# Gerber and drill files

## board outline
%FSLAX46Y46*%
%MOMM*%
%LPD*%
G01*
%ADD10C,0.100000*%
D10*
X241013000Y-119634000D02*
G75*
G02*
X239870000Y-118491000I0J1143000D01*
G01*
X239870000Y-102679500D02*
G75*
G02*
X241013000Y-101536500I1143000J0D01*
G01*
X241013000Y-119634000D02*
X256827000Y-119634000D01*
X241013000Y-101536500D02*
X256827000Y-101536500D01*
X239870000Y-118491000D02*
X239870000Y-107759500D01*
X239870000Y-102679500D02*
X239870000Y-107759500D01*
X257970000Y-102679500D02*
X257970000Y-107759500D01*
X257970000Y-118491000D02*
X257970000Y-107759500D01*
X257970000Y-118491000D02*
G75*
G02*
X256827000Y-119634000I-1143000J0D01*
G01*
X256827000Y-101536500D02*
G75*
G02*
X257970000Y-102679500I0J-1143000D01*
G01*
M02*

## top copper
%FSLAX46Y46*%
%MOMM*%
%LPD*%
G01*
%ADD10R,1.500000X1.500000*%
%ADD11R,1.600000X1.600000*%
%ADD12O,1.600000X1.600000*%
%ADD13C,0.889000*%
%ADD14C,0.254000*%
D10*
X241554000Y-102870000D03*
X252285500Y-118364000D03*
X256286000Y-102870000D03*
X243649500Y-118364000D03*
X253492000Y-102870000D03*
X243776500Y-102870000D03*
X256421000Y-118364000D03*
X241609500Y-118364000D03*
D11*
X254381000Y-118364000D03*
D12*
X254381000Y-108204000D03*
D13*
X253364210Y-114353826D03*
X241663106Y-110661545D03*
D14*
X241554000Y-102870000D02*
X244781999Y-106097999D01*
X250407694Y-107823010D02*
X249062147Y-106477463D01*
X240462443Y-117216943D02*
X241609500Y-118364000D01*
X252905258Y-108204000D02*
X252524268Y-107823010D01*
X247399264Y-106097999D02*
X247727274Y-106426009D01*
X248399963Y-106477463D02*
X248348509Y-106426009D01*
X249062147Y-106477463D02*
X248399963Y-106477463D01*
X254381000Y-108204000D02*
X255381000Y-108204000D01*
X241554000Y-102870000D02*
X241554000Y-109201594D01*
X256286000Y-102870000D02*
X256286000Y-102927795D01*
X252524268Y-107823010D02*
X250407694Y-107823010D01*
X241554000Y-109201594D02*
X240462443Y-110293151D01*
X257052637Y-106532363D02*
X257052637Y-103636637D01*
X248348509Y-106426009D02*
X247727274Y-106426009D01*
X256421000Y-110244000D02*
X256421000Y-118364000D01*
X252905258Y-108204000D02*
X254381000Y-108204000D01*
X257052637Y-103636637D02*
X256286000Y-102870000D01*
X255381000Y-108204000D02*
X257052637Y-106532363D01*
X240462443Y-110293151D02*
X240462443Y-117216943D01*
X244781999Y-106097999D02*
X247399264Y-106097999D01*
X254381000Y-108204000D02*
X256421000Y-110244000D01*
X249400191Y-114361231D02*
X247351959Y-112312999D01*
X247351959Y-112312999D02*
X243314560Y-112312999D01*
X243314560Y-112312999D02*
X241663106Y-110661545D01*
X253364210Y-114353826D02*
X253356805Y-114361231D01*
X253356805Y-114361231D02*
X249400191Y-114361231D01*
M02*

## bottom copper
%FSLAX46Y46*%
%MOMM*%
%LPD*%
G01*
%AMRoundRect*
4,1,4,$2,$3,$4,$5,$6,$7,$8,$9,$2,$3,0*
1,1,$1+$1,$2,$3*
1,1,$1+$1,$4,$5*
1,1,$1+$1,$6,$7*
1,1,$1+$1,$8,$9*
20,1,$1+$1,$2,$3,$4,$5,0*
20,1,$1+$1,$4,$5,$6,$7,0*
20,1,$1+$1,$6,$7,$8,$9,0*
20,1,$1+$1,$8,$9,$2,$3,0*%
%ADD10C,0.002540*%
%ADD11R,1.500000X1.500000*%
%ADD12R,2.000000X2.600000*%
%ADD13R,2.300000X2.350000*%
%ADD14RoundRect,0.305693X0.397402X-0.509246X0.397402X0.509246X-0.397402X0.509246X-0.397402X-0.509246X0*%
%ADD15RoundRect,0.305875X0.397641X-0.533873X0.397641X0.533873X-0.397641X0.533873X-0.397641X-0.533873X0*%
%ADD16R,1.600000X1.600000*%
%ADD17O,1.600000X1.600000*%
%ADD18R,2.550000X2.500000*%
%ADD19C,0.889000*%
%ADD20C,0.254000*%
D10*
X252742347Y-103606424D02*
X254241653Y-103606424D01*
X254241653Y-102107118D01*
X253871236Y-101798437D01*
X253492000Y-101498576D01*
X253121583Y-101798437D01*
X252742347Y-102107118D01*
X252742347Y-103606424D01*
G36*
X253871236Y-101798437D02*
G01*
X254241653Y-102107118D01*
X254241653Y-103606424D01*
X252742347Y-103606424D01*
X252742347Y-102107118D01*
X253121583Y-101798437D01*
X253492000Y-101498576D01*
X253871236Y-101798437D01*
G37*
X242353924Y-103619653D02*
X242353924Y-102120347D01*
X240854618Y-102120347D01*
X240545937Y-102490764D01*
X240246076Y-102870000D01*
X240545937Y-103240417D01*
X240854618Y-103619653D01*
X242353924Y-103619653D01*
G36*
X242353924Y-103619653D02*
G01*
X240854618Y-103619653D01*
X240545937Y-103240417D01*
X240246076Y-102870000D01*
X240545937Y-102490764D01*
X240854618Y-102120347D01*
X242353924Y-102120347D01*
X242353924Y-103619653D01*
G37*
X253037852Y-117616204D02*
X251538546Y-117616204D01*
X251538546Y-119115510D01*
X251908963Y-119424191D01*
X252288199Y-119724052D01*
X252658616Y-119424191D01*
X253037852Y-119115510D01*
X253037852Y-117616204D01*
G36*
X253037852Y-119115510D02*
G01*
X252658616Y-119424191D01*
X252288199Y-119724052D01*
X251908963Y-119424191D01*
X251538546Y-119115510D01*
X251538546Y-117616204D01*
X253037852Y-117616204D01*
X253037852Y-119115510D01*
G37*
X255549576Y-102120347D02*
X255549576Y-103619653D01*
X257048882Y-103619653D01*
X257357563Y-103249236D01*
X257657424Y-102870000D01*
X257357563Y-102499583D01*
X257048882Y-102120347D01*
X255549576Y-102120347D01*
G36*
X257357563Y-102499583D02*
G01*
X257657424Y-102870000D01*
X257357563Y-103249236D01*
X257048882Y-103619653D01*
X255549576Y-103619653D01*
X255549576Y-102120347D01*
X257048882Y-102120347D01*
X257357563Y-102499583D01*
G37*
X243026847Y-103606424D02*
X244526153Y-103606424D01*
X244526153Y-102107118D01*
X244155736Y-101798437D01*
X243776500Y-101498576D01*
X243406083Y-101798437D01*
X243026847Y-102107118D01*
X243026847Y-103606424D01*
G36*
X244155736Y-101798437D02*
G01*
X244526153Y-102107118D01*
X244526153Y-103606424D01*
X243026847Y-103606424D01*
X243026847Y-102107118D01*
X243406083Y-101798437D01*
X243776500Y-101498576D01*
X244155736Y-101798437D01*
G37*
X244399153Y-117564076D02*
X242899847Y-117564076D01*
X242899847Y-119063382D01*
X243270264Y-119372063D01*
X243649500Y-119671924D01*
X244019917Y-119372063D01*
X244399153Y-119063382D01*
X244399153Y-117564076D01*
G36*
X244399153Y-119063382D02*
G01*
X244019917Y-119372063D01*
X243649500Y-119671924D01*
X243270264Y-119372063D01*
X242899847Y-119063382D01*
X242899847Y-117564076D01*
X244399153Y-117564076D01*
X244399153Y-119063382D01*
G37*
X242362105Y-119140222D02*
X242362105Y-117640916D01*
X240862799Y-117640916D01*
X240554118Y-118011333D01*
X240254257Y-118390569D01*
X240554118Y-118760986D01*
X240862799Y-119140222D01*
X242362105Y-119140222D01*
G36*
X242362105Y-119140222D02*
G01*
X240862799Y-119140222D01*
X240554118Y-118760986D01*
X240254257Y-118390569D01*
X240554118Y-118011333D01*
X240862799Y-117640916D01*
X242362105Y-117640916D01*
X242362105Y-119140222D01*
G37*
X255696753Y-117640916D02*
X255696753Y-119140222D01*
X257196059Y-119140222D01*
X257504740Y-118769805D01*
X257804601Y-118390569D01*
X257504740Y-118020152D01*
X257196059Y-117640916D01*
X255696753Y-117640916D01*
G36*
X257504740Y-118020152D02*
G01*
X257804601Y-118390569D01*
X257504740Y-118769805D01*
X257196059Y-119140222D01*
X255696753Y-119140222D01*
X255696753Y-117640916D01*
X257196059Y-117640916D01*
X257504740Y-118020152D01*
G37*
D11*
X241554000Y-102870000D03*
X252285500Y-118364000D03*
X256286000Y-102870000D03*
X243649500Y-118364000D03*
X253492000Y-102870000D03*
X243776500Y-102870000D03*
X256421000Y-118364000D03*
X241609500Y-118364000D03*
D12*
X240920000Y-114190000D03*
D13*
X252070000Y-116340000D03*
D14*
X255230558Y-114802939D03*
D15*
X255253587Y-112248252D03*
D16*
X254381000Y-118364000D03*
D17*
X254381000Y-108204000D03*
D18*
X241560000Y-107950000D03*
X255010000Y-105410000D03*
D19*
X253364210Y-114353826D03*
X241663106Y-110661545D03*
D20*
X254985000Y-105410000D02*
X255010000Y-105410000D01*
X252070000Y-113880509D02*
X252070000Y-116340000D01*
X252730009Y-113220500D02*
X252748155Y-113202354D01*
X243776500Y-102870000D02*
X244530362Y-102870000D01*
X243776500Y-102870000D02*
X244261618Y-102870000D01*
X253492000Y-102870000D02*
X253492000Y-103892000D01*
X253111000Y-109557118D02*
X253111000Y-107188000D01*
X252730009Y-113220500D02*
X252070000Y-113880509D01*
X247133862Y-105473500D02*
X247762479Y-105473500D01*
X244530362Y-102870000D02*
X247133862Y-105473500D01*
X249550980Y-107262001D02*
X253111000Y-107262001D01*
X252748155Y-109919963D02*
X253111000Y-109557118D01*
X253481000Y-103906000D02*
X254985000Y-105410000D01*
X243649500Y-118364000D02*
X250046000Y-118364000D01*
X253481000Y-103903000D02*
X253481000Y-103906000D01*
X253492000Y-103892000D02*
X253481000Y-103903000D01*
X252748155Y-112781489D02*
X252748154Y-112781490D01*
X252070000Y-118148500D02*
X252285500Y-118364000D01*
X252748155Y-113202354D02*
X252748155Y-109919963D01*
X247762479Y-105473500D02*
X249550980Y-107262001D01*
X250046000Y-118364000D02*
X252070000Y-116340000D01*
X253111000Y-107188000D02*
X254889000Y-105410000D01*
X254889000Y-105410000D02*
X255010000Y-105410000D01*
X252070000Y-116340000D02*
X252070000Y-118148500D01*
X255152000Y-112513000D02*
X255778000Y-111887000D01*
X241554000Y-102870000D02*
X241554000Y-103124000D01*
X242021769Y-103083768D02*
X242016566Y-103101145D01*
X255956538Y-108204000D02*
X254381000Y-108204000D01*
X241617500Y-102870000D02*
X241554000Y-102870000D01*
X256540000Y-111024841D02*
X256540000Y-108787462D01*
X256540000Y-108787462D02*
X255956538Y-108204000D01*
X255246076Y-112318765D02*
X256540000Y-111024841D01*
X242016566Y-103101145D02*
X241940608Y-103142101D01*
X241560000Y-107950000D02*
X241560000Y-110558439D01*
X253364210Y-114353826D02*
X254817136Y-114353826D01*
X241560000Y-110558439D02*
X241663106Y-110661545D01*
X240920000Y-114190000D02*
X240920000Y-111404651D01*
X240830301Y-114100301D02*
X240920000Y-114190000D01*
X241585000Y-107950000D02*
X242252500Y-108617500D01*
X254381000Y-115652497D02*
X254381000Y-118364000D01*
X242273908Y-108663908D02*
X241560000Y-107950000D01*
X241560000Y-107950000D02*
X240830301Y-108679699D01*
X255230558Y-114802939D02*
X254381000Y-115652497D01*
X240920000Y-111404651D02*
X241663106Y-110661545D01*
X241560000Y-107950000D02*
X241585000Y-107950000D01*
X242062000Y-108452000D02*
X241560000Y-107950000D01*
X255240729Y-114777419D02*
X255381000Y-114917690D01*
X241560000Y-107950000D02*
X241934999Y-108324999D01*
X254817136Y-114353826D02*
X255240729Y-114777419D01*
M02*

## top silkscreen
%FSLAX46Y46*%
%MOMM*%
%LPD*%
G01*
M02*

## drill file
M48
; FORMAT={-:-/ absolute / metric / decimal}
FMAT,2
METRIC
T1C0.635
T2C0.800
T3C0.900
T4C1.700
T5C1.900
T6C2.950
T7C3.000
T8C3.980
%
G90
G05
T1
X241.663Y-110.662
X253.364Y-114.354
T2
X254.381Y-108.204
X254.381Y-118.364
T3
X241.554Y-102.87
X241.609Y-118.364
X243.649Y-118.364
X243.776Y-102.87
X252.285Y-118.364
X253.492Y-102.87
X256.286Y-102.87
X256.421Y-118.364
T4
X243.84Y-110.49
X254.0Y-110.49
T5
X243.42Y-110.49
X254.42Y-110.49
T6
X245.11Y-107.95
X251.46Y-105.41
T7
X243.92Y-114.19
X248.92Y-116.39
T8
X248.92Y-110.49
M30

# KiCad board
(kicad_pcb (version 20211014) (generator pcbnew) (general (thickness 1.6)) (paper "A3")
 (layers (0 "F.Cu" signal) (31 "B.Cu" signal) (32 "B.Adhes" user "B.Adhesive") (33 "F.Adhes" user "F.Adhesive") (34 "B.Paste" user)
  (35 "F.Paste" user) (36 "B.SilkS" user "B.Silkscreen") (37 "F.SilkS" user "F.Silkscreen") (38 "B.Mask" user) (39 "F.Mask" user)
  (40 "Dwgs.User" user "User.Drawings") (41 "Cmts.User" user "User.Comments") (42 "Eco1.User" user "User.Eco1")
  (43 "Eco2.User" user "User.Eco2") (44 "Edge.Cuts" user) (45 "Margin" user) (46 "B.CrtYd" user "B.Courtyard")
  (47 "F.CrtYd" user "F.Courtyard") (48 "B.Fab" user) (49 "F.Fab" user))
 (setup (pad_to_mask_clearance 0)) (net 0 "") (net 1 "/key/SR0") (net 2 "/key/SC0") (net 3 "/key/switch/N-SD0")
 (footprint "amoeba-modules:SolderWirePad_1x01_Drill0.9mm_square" (layer "F.Cu") (at 241.554 102.87)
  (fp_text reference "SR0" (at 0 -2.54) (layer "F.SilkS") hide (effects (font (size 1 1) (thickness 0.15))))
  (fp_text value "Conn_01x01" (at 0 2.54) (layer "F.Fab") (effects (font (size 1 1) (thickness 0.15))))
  (pad "1" thru_hole rect locked (at 0 0) (size 1.5 1.5) (drill 0.9) (layers *.Cu *.Mask) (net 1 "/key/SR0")))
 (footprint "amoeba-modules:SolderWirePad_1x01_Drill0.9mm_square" (layer "F.Cu") (at 252.2855 118.364)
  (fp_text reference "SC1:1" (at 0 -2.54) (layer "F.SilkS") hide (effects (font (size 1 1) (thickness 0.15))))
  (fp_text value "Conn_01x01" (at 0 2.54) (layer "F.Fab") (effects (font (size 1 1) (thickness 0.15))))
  (pad "1" thru_hole rect locked (at 0 0) (size 1.5 1.5) (drill 0.9) (layers *.Cu *.Mask) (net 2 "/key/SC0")))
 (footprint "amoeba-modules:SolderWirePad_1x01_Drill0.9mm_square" (layer "F.Cu") (at 256.286 102.87)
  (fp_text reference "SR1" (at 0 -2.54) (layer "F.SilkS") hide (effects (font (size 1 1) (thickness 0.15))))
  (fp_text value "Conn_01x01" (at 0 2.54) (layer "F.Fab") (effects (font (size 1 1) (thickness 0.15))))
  (pad "1" thru_hole rect locked (at 0 0) (size 1.5 1.5) (drill 0.9) (layers *.Cu *.Mask) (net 1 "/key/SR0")))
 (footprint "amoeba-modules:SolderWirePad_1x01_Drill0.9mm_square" (layer "F.Cu") (at 243.6495 118.364)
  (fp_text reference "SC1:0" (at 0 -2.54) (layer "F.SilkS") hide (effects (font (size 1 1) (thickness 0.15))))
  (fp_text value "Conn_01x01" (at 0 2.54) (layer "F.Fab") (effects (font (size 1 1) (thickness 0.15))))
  (pad "1" thru_hole rect locked (at 0 0) (size 1.5 1.5) (drill 0.9) (layers *.Cu *.Mask) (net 2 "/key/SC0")))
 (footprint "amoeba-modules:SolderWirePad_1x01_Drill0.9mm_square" (layer "F.Cu") (at 253.492 102.87)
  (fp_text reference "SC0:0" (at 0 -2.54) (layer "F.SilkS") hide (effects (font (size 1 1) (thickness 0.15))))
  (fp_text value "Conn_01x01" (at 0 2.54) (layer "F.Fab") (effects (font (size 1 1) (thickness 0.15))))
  (pad "1" thru_hole rect locked (at 0 0) (size 1.5 1.5) (drill 0.9) (layers *.Cu *.Mask) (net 2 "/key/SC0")))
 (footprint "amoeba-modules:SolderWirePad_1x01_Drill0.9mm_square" (layer "F.Cu") (at 243.7765 102.87)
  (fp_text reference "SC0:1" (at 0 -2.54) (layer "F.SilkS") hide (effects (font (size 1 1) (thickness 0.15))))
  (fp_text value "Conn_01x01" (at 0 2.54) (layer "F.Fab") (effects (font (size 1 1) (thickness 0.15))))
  (pad "1" thru_hole rect locked (at 0 0) (size 1.5 1.5) (drill 0.9) (layers *.Cu *.Mask) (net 2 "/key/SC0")))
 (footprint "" (layer "F.Cu") (at 256.921 118.364)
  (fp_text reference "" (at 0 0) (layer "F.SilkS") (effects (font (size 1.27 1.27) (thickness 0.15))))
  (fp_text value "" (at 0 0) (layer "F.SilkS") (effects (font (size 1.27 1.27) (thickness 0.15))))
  (pad "1" thru_hole rect locked (at -0.5 0) (size 1.5 1.5) (drill 0.9) (layers *.Cu *.Mask) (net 1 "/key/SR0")))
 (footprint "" (layer "F.Cu") (at 241.1095 118.364)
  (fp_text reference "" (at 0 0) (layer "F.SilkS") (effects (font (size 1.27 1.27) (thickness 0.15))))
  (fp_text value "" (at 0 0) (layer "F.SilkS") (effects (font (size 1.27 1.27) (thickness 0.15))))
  (pad "1" thru_hole rect locked (at 0.5 0) (size 1.5 1.5) (drill 0.9) (layers *.Cu *.Mask) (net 1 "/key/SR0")))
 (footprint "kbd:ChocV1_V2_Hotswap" (layer "F.Cu") (at 248.92 110.49)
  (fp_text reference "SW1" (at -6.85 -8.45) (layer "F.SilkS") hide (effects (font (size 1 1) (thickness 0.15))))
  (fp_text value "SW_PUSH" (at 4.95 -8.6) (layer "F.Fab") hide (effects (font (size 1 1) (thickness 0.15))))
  (pad "" np_thru_hole circle (at 5.5 0 90) (size 1.9 1.9) (drill 1.9) (layers *.Cu))
  (pad "" np_thru_hole circle (at -5 3.7 90) (size 3 3) (drill 3) (layers *.Cu *.Mask))
  (pad "" np_thru_hole circle (at 0 5.9 90) (size 3 3) (drill 3) (layers *.Cu *.Mask))
  (pad "" np_thru_hole circle (at -5.5 0 90) (size 1.9 1.9) (drill 1.9) (layers *.Cu))
  (pad "1" smd rect (at -8 3.7 180) (size 2 2.6) (layers "B.Cu" "B.Paste" "B.Mask") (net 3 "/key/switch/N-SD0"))
  (pad "2" smd rect (at 3.15 5.85 180) (size 2.3 2.35) (layers "B.Cu" "B.Paste" "B.Mask") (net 2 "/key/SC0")))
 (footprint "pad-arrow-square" (layer "B.Cu") (at 253.492 102.5525 90)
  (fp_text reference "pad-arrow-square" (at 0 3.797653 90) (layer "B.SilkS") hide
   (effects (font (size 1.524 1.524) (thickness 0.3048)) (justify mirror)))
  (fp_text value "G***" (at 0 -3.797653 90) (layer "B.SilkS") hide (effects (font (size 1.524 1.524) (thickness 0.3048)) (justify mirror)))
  (fp_poly
   (pts (xy -1.053924 -0.749653) (xy -1.053924 0.749653) (xy 0.445382 0.749653) (xy 0.754063 0.379236) (xy 1.053924 0)
    (xy 0.754063 -0.370417) (xy 0.445382 -0.749653) (xy -1.053924 -0.749653))
   (layer "B.Cu") (width 0.00254) (fill solid)))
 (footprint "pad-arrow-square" (layer "B.Cu") (at 241.3 102.87 180)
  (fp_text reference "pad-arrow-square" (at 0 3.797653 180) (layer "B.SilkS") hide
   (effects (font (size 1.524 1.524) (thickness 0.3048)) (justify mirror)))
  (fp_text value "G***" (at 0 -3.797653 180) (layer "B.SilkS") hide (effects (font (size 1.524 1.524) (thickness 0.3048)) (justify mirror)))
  (fp_poly
   (pts (xy -1.053924 -0.749653) (xy -1.053924 0.749653) (xy 0.445382 0.749653) (xy 0.754063 0.379236) (xy 1.053924 0)
    (xy 0.754063 -0.370417) (xy 0.445382 -0.749653) (xy -1.053924 -0.749653))
   (layer "B.Cu") (width 0.00254) (fill solid)))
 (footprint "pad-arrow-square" (layer "B.Cu") (at 252.288199 118.670128 -90)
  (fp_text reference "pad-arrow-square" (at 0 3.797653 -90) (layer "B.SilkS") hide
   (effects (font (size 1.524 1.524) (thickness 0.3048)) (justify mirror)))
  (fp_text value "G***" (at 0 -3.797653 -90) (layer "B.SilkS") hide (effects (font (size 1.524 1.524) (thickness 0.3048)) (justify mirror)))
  (fp_poly
   (pts (xy -1.053924 -0.749653) (xy -1.053924 0.749653) (xy 0.445382 0.749653) (xy 0.754063 0.379236) (xy 1.053924 0)
    (xy 0.754063 -0.370417) (xy 0.445382 -0.749653) (xy -1.053924 -0.749653))
   (layer "B.Cu") (width 0.00254) (fill solid)))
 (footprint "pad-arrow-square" (layer "B.Cu") (at 256.6035 102.87)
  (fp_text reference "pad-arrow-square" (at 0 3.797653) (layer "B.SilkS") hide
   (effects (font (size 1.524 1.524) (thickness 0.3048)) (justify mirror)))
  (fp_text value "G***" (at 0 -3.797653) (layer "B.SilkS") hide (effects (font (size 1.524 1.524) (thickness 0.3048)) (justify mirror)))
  (fp_poly
   (pts (xy -1.053924 -0.749653) (xy -1.053924 0.749653) (xy 0.445382 0.749653) (xy 0.754063 0.379236) (xy 1.053924 0)
    (xy 0.754063 -0.370417) (xy 0.445382 -0.749653) (xy -1.053924 -0.749653))
   (layer "B.Cu") (width 0.00254) (fill solid)))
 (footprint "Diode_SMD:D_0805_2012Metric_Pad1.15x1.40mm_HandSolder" (layer "B.Cu") (at 255.254 113.538 90)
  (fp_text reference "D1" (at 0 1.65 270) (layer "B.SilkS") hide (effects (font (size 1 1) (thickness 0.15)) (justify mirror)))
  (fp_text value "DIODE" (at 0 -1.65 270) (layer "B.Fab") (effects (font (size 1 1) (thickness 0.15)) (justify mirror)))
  (pad "1" smd roundrect (at -1.264939 -0.023442 90) (size 1.629879 1.40619) (layers "B.Cu" "B.Paste" "B.Mask")
   (roundrect_rratio 0.2173909642) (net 3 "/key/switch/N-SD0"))
  (pad "2" smd roundrect (at 1.289748 -0.000413 90) (size 1.679496 1.407033) (layers "B.Cu" "B.Paste" "B.Mask")
   (roundrect_rratio 0.2173900683) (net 1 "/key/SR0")))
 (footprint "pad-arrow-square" (layer "B.Cu") (at 243.7765 102.5525 90)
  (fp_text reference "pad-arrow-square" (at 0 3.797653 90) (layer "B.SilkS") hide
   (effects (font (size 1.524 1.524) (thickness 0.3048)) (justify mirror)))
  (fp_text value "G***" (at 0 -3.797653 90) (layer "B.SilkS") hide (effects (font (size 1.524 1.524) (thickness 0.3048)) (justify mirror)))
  (fp_poly
   (pts (xy -1.053924 -0.749653) (xy -1.053924 0.749653) (xy 0.445382 0.749653) (xy 0.754063 0.379236) (xy 1.053924 0)
    (xy 0.754063 -0.370417) (xy 0.445382 -0.749653) (xy -1.053924 -0.749653))
   (layer "B.Cu") (width 0.00254) (fill solid)))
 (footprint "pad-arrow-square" (layer "B.Cu") (at 243.6495 118.618 -90)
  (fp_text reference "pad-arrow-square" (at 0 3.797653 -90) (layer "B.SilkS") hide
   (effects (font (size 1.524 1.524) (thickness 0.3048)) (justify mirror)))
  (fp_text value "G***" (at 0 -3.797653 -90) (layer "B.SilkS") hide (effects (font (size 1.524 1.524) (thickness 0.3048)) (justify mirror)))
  (fp_poly
   (pts (xy -1.053924 -0.749653) (xy -1.053924 0.749653) (xy 0.445382 0.749653) (xy 0.754063 0.379236) (xy 1.053924 0)
    (xy 0.754063 -0.370417) (xy 0.445382 -0.749653) (xy -1.053924 -0.749653))
   (layer "B.Cu") (width 0.00254) (fill solid)))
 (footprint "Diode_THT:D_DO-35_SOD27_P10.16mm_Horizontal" (layer "B.Cu") (at 254.381 118.364 90)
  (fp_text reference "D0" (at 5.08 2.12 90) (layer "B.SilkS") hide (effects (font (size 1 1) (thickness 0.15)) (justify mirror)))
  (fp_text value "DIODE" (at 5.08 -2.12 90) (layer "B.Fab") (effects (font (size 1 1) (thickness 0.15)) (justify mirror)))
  (pad "1" thru_hole rect (at 0 0 90) (size 1.6 1.6) (drill 0.8) (layers *.Cu *.Mask) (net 3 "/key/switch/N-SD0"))
  (pad "2" thru_hole oval (at 10.16 0 90) (size 1.6 1.6) (drill 0.8) (layers *.Cu *.Mask) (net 1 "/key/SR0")))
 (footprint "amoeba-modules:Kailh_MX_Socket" (layer "B.Cu") (at 248.92 110.49 180)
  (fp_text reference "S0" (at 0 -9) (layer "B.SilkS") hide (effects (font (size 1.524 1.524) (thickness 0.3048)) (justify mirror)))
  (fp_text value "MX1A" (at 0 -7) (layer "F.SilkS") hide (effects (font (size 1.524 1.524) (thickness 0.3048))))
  (pad "" np_thru_hole circle locked (at 3.81 2.54 180) (size 2.95 2.95) (drill 2.95) (layers *.Cu *.Mask))
  (pad "" np_thru_hole circle locked (at 0 0 180) (size 3.98018 3.98018) (drill 3.98018) (layers *.Cu *.Mask))
  (pad "" np_thru_hole circle locked (at -5.08 0 180) (size 1.7 1.7) (drill 1.7) (layers *.Cu *.Mask))
  (pad "" np_thru_hole circle locked (at 5.08 0 180) (size 1.7 1.7) (drill 1.7) (layers *.Cu *.Mask))
  (pad "" np_thru_hole circle locked (at -2.54 5.08 180) (size 2.95 2.95) (drill 2.95) (layers *.Cu *.Mask))
  (pad "1" smd rect locked (at 7.36 2.54 180) (size 2.55 2.5) (layers "B.Cu" "B.Paste" "B.Mask") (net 3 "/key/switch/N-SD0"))
  (pad "2" smd rect locked (at -6.09 5.08 180) (size 2.55 2.5) (layers "B.Cu" "B.Paste" "B.Mask") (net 2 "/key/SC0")))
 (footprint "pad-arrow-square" (layer "B.Cu") (at 241.308181 118.390569 180)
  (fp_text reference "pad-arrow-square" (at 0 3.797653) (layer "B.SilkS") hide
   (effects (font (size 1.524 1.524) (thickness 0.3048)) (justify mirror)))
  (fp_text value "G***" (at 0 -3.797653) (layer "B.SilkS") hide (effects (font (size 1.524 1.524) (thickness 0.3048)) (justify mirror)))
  (fp_poly
   (pts (xy -1.053924 -0.749653) (xy -1.053924 0.749653) (xy 0.445382 0.749653) (xy 0.754063 0.379236) (xy 1.053924 0)
    (xy 0.754063 -0.370417) (xy 0.445382 -0.749653) (xy -1.053924 -0.749653))
   (layer "B.Cu") (width 0.00254) (fill solid)))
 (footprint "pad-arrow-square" (layer "B.Cu") (at 256.750677 118.390569)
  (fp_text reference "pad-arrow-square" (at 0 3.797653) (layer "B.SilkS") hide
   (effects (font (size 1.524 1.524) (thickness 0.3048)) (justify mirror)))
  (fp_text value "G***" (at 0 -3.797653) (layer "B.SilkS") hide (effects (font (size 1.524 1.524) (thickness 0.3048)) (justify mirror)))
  (fp_poly
   (pts (xy -1.053924 -0.749653) (xy -1.053924 0.749653) (xy 0.445382 0.749653) (xy 0.754063 0.379236) (xy 1.053924 0)
    (xy 0.754063 -0.370417) (xy 0.445382 -0.749653) (xy -1.053924 -0.749653))
   (layer "B.Cu") (width 0.00254) (fill solid)))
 (gr_arc (start 241.013 119.634) (mid 240.204777 119.299223) (end 239.87 118.491) (layer "Edge.Cuts") (width 0.1))
 (gr_arc (start 239.87 102.6795) (mid 240.204777 101.871277) (end 241.013 101.5365) (layer "Edge.Cuts") (width 0.1))
 (gr_line (start 241.013 119.634) (end 256.827 119.634) (layer "Edge.Cuts") (width 0.1))
 (gr_line (start 241.013 101.5365) (end 256.827 101.5365) (layer "Edge.Cuts") (width 0.1))
 (gr_line (start 239.87 118.491) (end 239.87 107.7595) (layer "Edge.Cuts") (width 0.1))
 (gr_line (start 239.87 102.6795) (end 239.87 107.7595) (layer "Edge.Cuts") (width 0.1))
 (gr_line (start 257.97 102.6795) (end 257.97 107.7595) (layer "Edge.Cuts") (width 0.1))
 (gr_line (start 257.97 118.491) (end 257.97 107.7595) (layer "Edge.Cuts") (width 0.1))
 (gr_arc (start 257.97 118.491) (mid 257.635223 119.299223) (end 256.827 119.634) (layer "Edge.Cuts") (width 0.1))
 (gr_arc (start 256.827 101.5365) (mid 257.635223 101.871277) (end 257.97 102.6795) (layer "Edge.Cuts") (width 0.1))
 (segment (start 254.985 105.41) (end 255.01 105.41) (width 0.254) (layer "B.Cu") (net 2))
 (segment (start 252.07 113.880509) (end 252.07 116.34) (width 0.254) (layer "B.Cu") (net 2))
 (segment (start 252.730009 113.2205) (end 252.748155 113.202354) (width 0.254) (layer "B.Cu") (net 2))
 (segment (start 243.7765 102.87) (end 244.530362 102.87) (width 0.254) (layer "B.Cu") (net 2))
 (segment (start 243.7765 102.87) (end 244.261618 102.87) (width 0.254) (layer "B.Cu") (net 2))
 (segment (start 253.492 102.87) (end 253.492 103.892) (width 0.254) (layer "B.Cu") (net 2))
 (segment (start 253.111 109.557118) (end 253.111 107.188) (width 0.254) (layer "B.Cu") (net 2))
 (segment (start 252.730009 113.2205) (end 252.07 113.880509) (width 0.254) (layer "B.Cu") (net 2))
 (segment (start 247.133862 105.4735) (end 247.762479 105.4735) (width 0.254) (layer "B.Cu") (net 2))
 (segment (start 244.530362 102.87) (end 247.133862 105.4735) (width 0.254) (layer "B.Cu") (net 2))
 (segment (start 249.55098 107.262001) (end 253.111 107.262001) (width 0.254) (layer "B.Cu") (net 2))
 (segment (start 252.748155 109.919963) (end 253.111 109.557118) (width 0.254) (layer "B.Cu") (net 2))
 (segment (start 253.481 103.906) (end 254.985 105.41) (width 0.254) (layer "B.Cu") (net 2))
 (segment (start 243.6495 118.364) (end 250.046 118.364) (width 0.254) (layer "B.Cu") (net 2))
 (segment (start 253.481 103.903) (end 253.481 103.906) (width 0.254) (layer "B.Cu") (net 2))
 (segment (start 253.492 103.892) (end 253.481 103.903) (width 0.254) (layer "B.Cu") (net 2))
 (segment (start 252.748155 112.781489) (end 252.748154 112.78149) (width 0.254) (layer "B.Cu") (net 2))
 (segment (start 252.07 118.1485) (end 252.2855 118.364) (width 0.254) (layer "B.Cu") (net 2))
 (segment (start 252.748155 113.202354) (end 252.748155 109.919963) (width 0.254) (layer "B.Cu") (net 2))
 (segment (start 247.762479 105.4735) (end 249.55098 107.262001) (width 0.254) (layer "B.Cu") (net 2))
 (segment (start 250.046 118.364) (end 252.07 116.34) (width 0.254) (layer "B.Cu") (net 2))
 (segment (start 253.111 107.188) (end 254.889 105.41) (width 0.254) (layer "B.Cu") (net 2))
 (segment (start 254.889 105.41) (end 255.01 105.41) (width 0.254) (layer "B.Cu") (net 2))
 (segment (start 252.07 116.34) (end 252.07 118.1485) (width 0.254) (layer "B.Cu") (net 2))
 (segment (start 241.554 102.87) (end 244.781999 106.097999) (width 0.254) (layer "F.Cu") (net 1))
 (segment (start 250.407694 107.82301) (end 249.062147 106.477463) (width 0.254) (layer "F.Cu") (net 1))
 (segment (start 240.462443 117.216943) (end 241.6095 118.364) (width 0.254) (layer "F.Cu") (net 1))
 (segment (start 252.905258 108.204) (end 252.524268 107.82301) (width 0.254) (layer "F.Cu") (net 1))
 (segment (start 247.399264 106.097999) (end 247.727274 106.426009) (width 0.254) (layer "F.Cu") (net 1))
 (segment (start 248.399963 106.477463) (end 248.348509 106.426009) (width 0.254) (layer "F.Cu") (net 1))
 (segment (start 249.062147 106.477463) (end 248.399963 106.477463) (width 0.254) (layer "F.Cu") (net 1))
 (segment (start 254.381 108.204) (end 255.381 108.204) (width 0.254) (layer "F.Cu") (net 1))
 (segment (start 241.554 102.87) (end 241.554 109.201594) (width 0.254) (layer "F.Cu") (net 1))
 (segment (start 256.286 102.87) (end 256.286 102.927795) (width 0.254) (layer "F.Cu") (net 1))
 (segment (start 252.524268 107.82301) (end 250.407694 107.82301) (width 0.254) (layer "F.Cu") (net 1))
 (segment (start 241.554 109.201594) (end 240.462443 110.293151) (width 0.254) (layer "F.Cu") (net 1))
 (segment (start 257.052637 106.532363) (end 257.052637 103.636637) (width 0.254) (layer "F.Cu") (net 1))
 (segment (start 248.348509 106.426009) (end 247.727274 106.426009) (width 0.254) (layer "F.Cu") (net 1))
 (segment (start 256.421 110.244) (end 256.421 118.364) (width 0.254) (layer "F.Cu") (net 1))
 (segment (start 252.905258 108.204) (end 254.381 108.204) (width 0.254) (layer "F.Cu") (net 1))
 (segment (start 257.052637 103.636637) (end 256.286 102.87) (width 0.254) (layer "F.Cu") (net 1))
 (segment (start 255.381 108.204) (end 257.052637 106.532363) (width 0.254) (layer "F.Cu") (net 1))
 (segment (start 240.462443 110.293151) (end 240.462443 117.216943) (width 0.254) (layer "F.Cu") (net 1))
 (segment (start 244.781999 106.097999) (end 247.399264 106.097999) (width 0.254) (layer "F.Cu") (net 1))
 (segment (start 254.381 108.204) (end 256.421 110.244) (width 0.254) (layer "F.Cu") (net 1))
 (segment (start 255.152 112.513) (end 255.778 111.887) (width 0.254) (layer "B.Cu") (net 1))
 (segment (start 241.554 102.87) (end 241.554 103.124) (width 0.254) (layer "B.Cu") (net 1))
 (segment (start 242.021769 103.083768) (end 242.016566 103.101145) (width 0.254) (layer "B.Cu") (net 1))
 (segment (start 255.956538 108.204) (end 254.381 108.204) (width 0.254) (layer "B.Cu") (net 1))
 (segment (start 241.6175 102.87) (end 241.554 102.87) (width 0.254) (layer "B.Cu") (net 1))
 (segment (start 256.54 111.024841) (end 256.54 108.787462) (width 0.254) (layer "B.Cu") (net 1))
 (segment (start 256.54 108.787462) (end 255.956538 108.204) (width 0.254) (layer "B.Cu") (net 1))
 (segment (start 255.246076 112.318765) (end 256.54 111.024841) (width 0.254) (layer "B.Cu") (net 1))
 (segment (start 242.016566 103.101145) (end 241.940608 103.142101) (width 0.254) (layer "B.Cu") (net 1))
 (segment (start 249.400191 114.361231) (end 247.351959 112.312999) (width 0.254) (layer "F.Cu") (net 3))
 (segment (start 247.351959 112.312999) (end 243.31456 112.312999) (width 0.254) (layer "F.Cu") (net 3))
 (segment (start 243.31456 112.312999) (end 241.663106 110.661545) (width 0.254) (layer "F.Cu") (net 3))
 (segment (start 253.36421 114.353826) (end 253.356805 114.361231) (width 0.254) (layer "F.Cu") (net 3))
 (segment (start 253.356805 114.361231) (end 249.400191 114.361231) (width 0.254) (layer "F.Cu") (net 3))
 (via (at 253.36421 114.353826) (size 0.889) (drill 0.635) (layers "F.Cu" "B.Cu") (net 3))
 (via (at 241.663106 110.661545) (size 0.889) (drill 0.635) (layers "F.Cu" "B.Cu") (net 3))
 (segment (start 241.56 107.95) (end 241.56 110.558439) (width 0.254) (layer "B.Cu") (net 3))
 (segment (start 253.36421 114.353826) (end 254.817136 114.353826) (width 0.254) (layer "B.Cu") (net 3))
 (segment (start 241.56 110.558439) (end 241.663106 110.661545) (width 0.254) (layer "B.Cu") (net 3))
 (segment (start 240.92 114.19) (end 240.92 111.404651) (width 0.254) (layer "B.Cu") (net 3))
 (segment (start 240.830301 114.100301) (end 240.92 114.19) (width 0.254) (layer "B.Cu") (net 3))
 (segment (start 241.585 107.95) (end 242.2525 108.6175) (width 0.254) (layer "B.Cu") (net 3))
 (segment (start 254.381 115.652497) (end 254.381 118.364) (width 0.254) (layer "B.Cu") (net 3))
 (segment (start 242.273908 108.663908) (end 241.56 107.95) (width 0.254) (layer "B.Cu") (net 3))
 (segment (start 241.56 107.95) (end 240.830301 108.679699) (width 0.254) (layer "B.Cu") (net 3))
 (segment (start 255.230558 114.802939) (end 254.381 115.652497) (width 0.254) (layer "B.Cu") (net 3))
 (segment (start 240.92 111.404651) (end 241.663106 110.661545) (width 0.254) (layer "B.Cu") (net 3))
 (segment (start 241.56 107.95) (end 241.585 107.95) (width 0.254) (layer "B.Cu") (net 3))
 (segment (start 242.062 108.452) (end 241.56 107.95) (width 0.254) (layer "B.Cu") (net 3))
 (segment (start 255.240729 114.777419) (end 255.381 114.91769) (width 0.254) (layer "B.Cu") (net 3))
 (segment (start 241.56 107.95) (end 241.934999 108.324999) (width 0.254) (layer "B.Cu") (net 3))
 (segment (start 254.817136 114.353826) (end 255.240729 114.777419) (width 0.254) (layer "B.Cu") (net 3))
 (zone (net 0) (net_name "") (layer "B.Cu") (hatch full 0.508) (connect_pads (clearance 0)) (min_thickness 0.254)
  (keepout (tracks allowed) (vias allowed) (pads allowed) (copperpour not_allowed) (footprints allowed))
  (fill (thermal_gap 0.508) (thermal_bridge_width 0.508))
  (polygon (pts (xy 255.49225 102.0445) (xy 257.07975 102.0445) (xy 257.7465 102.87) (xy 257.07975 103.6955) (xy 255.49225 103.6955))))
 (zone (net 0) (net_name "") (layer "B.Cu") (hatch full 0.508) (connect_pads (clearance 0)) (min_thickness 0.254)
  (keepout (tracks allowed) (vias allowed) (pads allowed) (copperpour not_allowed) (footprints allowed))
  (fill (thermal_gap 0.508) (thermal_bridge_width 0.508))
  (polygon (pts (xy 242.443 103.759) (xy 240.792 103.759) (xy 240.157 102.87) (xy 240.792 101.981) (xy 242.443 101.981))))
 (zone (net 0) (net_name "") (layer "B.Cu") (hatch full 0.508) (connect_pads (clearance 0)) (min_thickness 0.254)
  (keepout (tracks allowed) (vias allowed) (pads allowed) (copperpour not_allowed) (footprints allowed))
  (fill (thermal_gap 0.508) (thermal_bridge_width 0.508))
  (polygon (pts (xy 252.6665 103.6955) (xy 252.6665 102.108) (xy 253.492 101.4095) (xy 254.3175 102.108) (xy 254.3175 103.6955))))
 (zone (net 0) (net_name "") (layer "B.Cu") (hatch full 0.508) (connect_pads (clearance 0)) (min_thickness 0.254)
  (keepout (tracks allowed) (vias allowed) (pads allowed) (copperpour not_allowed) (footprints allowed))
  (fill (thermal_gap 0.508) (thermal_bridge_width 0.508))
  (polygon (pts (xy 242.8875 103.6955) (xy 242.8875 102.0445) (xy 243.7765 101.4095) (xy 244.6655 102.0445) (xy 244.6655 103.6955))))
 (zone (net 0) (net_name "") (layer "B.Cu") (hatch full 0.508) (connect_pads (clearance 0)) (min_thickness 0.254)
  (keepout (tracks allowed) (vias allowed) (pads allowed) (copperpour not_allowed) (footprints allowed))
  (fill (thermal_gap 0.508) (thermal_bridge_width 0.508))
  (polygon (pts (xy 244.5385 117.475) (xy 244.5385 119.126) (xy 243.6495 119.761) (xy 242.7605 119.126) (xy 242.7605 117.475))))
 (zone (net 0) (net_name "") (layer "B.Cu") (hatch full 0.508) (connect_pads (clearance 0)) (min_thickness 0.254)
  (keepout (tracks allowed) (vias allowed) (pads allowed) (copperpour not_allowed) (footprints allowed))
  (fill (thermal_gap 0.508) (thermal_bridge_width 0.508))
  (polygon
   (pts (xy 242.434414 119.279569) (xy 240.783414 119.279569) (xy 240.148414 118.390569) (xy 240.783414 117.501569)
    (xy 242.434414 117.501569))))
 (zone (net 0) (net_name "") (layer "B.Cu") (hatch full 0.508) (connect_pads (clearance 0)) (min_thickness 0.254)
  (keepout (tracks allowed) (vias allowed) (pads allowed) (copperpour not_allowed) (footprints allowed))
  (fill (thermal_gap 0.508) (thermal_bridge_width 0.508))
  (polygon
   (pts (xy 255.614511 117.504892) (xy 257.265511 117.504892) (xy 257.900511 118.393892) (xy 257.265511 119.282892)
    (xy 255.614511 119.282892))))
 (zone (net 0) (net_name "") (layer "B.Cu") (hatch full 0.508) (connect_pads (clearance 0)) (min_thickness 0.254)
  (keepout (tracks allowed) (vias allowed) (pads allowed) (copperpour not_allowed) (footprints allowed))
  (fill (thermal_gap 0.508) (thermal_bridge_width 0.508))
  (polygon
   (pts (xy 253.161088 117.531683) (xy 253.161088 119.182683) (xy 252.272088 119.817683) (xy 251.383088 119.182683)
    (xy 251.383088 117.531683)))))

